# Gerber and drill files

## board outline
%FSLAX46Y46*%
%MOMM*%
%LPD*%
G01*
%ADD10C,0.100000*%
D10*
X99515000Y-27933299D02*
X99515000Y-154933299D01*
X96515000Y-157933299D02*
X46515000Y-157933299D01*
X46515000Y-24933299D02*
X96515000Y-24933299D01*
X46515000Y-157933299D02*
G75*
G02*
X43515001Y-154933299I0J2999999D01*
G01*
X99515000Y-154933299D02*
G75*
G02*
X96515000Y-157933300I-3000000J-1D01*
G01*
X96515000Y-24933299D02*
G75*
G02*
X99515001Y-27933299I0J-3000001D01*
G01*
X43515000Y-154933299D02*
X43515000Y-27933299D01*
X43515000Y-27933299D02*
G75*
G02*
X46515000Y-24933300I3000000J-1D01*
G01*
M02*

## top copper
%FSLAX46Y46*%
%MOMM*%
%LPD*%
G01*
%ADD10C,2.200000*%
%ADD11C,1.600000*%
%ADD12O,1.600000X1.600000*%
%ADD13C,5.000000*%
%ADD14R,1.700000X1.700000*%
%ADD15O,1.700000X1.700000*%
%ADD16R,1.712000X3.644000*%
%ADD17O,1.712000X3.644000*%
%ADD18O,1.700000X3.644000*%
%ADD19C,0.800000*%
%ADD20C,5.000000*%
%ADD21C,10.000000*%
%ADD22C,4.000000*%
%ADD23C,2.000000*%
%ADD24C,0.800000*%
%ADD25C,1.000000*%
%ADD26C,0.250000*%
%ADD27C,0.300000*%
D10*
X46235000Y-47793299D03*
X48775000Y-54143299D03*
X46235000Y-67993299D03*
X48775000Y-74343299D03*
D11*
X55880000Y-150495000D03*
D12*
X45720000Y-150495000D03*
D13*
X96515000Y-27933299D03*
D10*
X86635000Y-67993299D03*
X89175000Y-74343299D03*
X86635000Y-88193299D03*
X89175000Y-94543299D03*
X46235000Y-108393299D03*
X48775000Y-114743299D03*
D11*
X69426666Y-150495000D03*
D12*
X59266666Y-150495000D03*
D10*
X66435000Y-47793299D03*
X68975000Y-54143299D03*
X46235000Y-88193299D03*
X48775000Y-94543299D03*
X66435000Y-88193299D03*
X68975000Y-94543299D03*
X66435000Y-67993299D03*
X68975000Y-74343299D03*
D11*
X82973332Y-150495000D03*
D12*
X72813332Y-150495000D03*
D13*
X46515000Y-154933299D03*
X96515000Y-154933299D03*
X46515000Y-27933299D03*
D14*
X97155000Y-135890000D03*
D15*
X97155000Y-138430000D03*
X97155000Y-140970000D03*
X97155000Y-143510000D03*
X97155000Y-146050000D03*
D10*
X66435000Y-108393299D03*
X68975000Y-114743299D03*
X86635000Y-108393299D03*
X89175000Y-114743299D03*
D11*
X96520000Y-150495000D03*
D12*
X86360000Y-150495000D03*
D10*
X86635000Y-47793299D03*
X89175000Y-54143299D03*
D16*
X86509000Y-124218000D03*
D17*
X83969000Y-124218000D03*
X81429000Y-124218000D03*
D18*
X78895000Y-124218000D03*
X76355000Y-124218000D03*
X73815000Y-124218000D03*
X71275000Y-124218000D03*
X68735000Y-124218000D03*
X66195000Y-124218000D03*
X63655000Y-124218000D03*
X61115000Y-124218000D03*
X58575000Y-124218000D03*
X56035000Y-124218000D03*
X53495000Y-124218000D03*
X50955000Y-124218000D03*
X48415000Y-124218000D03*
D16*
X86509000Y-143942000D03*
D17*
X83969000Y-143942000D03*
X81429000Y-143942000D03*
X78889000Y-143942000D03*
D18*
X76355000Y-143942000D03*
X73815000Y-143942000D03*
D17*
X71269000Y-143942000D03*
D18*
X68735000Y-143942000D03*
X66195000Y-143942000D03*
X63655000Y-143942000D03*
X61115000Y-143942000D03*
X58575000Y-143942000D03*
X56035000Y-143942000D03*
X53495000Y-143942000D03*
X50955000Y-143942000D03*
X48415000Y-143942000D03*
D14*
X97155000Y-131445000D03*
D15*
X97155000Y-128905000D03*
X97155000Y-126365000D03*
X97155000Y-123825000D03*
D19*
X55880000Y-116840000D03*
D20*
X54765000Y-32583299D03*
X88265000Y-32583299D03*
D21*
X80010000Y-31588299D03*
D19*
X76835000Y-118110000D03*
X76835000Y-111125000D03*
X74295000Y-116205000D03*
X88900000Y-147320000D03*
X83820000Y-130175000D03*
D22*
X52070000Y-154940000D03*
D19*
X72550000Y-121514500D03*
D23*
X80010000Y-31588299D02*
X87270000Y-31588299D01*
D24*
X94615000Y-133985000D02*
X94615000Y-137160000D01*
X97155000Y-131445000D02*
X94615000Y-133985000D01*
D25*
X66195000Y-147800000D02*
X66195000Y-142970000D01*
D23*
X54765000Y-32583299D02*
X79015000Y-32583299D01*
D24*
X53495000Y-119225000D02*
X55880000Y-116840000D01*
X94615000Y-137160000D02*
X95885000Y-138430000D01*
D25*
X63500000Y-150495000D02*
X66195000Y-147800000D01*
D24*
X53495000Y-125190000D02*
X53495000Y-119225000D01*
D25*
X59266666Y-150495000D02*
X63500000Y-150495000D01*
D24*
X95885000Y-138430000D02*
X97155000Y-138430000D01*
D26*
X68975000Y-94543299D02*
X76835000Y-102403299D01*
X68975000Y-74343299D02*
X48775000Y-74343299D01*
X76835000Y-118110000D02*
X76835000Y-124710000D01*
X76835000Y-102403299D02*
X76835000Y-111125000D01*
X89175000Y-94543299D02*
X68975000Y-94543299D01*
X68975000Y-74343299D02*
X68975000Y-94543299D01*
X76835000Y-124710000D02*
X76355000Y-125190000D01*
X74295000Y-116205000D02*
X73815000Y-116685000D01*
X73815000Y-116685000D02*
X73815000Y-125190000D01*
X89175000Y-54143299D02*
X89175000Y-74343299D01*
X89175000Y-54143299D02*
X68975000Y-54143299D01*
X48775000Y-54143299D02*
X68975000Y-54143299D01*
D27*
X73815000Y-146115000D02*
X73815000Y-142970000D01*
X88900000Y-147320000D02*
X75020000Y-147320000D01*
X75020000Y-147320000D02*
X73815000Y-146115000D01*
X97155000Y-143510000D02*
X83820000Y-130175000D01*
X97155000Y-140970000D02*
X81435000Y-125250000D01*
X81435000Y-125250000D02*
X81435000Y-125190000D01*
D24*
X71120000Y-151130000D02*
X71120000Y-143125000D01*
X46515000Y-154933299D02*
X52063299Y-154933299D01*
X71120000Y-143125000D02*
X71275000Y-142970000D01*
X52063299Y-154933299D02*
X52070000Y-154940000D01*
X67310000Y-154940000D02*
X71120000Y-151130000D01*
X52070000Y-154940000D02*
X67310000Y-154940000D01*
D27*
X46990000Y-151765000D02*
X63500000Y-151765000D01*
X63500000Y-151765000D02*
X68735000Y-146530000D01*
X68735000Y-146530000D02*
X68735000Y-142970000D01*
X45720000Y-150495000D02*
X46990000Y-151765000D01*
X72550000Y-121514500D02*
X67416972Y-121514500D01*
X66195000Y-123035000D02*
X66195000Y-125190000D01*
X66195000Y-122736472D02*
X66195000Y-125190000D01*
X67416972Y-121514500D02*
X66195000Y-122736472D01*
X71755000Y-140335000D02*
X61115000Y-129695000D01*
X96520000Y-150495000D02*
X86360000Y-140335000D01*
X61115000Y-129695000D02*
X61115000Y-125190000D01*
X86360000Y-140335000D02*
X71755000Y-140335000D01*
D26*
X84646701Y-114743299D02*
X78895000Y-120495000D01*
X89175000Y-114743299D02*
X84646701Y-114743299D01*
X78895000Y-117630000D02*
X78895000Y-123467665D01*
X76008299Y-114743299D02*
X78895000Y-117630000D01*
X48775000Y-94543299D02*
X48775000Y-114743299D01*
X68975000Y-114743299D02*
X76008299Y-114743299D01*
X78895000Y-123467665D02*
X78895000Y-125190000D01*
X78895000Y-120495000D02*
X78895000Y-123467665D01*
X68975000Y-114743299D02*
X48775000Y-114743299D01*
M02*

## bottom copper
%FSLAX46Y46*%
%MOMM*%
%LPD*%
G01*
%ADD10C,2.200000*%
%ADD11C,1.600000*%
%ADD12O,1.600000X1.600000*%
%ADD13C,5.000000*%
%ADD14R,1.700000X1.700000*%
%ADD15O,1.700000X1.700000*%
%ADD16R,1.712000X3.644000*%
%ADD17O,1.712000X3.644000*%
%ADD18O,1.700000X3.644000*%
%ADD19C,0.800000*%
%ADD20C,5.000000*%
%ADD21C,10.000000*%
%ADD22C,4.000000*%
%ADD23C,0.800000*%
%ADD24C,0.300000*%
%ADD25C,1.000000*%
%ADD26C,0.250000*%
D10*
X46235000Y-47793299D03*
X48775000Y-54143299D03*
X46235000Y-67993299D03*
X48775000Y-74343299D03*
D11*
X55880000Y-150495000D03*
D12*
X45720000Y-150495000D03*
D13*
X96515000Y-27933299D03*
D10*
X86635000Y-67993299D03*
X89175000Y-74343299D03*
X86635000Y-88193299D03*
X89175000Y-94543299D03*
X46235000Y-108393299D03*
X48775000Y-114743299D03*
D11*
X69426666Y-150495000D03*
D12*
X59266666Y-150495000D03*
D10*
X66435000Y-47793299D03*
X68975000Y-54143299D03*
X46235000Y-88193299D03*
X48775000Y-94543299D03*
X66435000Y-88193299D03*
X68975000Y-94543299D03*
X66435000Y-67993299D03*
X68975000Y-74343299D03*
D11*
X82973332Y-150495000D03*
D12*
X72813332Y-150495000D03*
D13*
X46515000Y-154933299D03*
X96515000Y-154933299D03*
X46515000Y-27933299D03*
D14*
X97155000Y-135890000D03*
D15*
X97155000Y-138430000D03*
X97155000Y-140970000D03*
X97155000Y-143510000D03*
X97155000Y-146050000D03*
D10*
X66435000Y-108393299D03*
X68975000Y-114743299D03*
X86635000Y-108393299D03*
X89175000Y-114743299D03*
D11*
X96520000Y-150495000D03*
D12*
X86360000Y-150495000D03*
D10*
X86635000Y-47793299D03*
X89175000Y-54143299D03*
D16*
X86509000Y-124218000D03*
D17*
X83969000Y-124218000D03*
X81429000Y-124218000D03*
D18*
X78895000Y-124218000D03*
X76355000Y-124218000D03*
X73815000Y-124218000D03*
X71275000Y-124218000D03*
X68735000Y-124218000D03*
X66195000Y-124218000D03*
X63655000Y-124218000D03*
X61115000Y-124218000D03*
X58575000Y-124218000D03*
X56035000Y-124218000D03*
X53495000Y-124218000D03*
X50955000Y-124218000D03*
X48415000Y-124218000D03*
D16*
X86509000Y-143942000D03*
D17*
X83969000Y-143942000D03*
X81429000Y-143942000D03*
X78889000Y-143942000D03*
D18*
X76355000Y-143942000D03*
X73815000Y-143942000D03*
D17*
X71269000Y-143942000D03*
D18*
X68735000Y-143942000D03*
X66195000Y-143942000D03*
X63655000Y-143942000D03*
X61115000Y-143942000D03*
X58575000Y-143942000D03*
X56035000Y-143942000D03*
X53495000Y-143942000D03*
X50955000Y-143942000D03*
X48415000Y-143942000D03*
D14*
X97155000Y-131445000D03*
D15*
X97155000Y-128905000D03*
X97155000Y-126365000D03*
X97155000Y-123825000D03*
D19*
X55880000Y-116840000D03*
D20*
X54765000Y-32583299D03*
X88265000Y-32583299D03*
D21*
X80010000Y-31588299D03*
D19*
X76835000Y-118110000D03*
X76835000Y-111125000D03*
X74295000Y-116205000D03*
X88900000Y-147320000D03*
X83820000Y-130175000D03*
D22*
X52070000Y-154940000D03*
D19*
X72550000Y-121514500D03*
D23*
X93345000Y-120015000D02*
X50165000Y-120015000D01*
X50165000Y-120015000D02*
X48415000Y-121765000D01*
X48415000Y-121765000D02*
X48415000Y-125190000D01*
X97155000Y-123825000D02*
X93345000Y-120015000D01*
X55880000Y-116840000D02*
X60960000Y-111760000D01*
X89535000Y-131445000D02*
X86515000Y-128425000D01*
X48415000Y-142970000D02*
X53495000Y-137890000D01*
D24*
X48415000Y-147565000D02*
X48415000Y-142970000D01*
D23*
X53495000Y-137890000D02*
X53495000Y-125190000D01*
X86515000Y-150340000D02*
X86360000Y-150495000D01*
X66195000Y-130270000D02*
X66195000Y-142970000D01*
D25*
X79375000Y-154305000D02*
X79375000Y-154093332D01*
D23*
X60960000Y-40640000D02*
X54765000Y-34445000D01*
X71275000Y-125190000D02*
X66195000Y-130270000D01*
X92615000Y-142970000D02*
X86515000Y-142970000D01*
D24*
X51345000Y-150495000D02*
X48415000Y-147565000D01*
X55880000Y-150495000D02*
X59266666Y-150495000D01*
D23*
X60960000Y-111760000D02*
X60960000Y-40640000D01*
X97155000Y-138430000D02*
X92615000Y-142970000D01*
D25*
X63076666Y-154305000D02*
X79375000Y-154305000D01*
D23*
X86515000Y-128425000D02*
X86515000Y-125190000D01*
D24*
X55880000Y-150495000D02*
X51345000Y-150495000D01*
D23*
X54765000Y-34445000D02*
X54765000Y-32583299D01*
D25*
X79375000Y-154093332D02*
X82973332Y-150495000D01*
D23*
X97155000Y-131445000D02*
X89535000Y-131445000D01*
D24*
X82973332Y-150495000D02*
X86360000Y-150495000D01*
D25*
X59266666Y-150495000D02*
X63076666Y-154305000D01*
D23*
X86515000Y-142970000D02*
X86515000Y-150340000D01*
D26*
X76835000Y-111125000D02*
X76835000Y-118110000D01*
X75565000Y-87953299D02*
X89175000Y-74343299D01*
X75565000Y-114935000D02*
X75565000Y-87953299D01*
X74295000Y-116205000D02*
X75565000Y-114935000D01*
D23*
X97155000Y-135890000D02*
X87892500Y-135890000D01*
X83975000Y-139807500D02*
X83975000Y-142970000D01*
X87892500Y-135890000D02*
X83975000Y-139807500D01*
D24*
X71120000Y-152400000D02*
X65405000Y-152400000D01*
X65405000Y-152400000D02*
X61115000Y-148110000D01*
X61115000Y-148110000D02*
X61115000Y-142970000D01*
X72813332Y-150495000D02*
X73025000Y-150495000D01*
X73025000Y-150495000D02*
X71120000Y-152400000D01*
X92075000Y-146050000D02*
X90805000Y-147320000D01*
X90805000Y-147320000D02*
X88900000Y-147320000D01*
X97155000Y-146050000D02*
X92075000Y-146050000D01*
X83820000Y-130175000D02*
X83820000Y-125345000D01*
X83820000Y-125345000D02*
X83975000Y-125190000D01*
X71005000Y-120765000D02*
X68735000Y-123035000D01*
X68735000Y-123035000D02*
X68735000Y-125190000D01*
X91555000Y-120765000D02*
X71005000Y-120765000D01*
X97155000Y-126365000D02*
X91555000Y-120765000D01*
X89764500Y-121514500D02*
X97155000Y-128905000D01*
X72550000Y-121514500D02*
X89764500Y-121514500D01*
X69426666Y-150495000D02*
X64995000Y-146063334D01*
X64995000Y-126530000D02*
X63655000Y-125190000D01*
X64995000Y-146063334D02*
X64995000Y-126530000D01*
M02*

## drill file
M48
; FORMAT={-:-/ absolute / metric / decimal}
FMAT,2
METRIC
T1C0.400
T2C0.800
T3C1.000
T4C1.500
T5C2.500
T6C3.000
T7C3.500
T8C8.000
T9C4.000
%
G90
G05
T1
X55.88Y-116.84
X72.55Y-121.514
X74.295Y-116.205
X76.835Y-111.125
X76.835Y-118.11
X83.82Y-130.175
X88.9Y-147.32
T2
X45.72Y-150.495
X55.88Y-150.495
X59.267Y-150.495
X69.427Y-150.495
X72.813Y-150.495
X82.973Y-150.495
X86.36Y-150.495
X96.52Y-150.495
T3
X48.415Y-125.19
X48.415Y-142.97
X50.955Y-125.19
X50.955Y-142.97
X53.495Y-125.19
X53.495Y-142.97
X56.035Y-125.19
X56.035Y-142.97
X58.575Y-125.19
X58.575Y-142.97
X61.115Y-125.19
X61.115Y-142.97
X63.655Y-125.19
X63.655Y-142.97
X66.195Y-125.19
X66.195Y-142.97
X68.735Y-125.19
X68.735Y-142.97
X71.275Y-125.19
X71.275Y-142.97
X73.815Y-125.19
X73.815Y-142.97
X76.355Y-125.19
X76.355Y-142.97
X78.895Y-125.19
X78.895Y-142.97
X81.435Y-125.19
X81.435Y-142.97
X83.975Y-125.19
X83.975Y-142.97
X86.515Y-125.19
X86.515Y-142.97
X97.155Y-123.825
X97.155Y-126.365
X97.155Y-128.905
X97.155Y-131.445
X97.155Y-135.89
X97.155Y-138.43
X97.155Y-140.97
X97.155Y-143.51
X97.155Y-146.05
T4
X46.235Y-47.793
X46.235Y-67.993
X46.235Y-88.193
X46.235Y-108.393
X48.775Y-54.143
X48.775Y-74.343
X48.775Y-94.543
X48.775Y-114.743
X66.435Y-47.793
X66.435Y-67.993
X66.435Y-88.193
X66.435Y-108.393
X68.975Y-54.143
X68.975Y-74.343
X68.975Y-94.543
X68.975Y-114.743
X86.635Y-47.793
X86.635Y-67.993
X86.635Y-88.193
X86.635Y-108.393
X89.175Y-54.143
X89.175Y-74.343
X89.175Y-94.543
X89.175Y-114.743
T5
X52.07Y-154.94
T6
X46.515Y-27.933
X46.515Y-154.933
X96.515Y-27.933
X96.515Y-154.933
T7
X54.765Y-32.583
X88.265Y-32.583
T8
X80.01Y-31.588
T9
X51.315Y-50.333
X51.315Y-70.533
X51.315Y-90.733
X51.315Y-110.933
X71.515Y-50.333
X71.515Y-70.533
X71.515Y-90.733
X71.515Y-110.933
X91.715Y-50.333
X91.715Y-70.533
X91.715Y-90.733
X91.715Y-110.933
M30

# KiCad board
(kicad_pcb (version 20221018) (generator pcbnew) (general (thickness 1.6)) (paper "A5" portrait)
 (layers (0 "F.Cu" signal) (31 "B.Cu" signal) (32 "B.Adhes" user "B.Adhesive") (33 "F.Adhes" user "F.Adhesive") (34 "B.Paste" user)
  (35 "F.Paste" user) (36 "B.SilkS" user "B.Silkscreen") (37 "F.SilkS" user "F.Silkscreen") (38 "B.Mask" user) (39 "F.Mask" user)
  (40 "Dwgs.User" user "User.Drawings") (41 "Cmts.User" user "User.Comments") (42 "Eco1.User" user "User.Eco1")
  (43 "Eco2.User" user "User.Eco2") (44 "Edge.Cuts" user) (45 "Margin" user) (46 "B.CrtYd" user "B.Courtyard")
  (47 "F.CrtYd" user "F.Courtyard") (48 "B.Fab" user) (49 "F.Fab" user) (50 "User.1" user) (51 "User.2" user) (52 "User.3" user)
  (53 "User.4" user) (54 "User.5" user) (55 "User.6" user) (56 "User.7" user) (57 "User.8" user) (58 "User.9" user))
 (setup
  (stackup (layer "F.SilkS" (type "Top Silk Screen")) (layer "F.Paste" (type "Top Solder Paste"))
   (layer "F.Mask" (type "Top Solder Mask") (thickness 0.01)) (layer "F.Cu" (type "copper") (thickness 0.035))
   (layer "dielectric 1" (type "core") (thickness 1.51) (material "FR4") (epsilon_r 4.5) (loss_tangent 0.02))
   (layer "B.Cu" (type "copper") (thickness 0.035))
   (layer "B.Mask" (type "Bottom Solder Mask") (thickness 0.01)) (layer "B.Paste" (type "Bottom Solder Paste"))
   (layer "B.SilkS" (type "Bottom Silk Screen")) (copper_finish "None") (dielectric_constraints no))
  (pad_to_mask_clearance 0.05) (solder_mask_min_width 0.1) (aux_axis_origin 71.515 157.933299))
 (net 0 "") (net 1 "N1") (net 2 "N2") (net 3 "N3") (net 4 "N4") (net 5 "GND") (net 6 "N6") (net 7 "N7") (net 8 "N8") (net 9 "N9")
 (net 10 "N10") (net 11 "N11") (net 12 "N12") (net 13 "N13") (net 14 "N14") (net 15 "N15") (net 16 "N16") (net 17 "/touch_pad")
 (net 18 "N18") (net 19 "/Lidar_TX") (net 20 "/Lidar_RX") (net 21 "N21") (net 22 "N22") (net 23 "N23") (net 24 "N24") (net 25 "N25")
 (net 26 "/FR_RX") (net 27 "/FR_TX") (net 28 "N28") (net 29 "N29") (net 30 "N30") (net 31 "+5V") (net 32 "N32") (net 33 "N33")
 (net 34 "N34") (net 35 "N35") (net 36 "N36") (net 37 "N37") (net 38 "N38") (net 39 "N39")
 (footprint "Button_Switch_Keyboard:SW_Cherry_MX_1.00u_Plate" (layer "F.Cu") (at 46.235 47.793299 90)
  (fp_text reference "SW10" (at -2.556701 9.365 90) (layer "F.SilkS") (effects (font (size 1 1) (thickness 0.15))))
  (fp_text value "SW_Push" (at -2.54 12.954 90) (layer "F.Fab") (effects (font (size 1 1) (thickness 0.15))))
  (pad "" np_thru_hole circle (at -2.54 5.08 90) (size 4 4) (drill 4) (layers "*.Cu" "*.Mask"))
  (pad "1" thru_hole circle (at 0 0 90) (size 2.2 2.2) (drill 1.5) (layers "*.Cu" "*.Mask") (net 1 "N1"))
  (pad "2" thru_hole circle (at -6.35 2.54 90) (size 2.2 2.2) (drill 1.5) (layers "*.Cu" "*.Mask") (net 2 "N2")))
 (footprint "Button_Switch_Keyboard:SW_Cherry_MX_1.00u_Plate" (layer "F.Cu") (at 46.235 67.993299 90)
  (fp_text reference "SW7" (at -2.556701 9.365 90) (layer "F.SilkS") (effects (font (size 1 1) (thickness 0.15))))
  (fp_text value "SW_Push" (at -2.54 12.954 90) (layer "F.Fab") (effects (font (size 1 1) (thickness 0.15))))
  (pad "" np_thru_hole circle (at -2.54 5.08 90) (size 4 4) (drill 4) (layers "*.Cu" "*.Mask"))
  (pad "1" thru_hole circle (at 0 0 90) (size 2.2 2.2) (drill 1.5) (layers "*.Cu" "*.Mask") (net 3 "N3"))
  (pad "2" thru_hole circle (at -6.35 2.54 90) (size 2.2 2.2) (drill 1.5) (layers "*.Cu" "*.Mask") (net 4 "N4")))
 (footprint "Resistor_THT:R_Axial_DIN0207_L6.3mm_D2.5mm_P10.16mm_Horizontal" (layer "F.Cu") (at 55.88 150.495 180)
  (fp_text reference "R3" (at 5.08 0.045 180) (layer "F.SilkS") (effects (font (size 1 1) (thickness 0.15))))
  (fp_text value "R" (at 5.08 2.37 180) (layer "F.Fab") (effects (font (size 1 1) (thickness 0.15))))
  (pad "1" thru_hole circle (at 0 0 180) (size 1.6 1.6) (drill 0.8) (layers "*.Cu" "*.Mask") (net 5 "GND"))
  (pad "2" thru_hole oval (at 10.16 0 180) (size 1.6 1.6) (drill 0.8) (layers "*.Cu" "*.Mask") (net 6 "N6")))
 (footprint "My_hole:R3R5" (layer "F.Cu") (at 96.52 27.763299)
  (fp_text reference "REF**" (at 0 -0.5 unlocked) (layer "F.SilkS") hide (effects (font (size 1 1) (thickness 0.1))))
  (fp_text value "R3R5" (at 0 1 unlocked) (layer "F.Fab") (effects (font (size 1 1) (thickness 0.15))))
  (pad "1" thru_hole circle (at -0.005 0.17 180) (size 5 5) (drill 3) (layers "*.Cu" "*.Mask") (remove_unused_layers) (keep_end_layers)
   (zone_layer_connections)))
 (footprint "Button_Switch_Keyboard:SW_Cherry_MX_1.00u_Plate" (layer "F.Cu") (at 86.635 67.993299 90)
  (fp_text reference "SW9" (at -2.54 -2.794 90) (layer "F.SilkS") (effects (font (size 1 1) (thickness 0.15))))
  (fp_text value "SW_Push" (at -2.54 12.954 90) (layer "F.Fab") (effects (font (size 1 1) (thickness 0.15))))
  (pad "" np_thru_hole circle (at -2.54 5.08 90) (size 4 4) (drill 4) (layers "*.Cu" "*.Mask"))
  (pad "1" thru_hole circle (at 0 0 90) (size 2.2 2.2) (drill 1.5) (layers "*.Cu" "*.Mask") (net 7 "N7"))
  (pad "2" thru_hole circle (at -6.35 2.54 90) (size 2.2 2.2) (drill 1.5) (layers "*.Cu" "*.Mask") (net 2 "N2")))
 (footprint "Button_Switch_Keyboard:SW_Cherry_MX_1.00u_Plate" (layer "F.Cu") (at 86.635 88.193299 90)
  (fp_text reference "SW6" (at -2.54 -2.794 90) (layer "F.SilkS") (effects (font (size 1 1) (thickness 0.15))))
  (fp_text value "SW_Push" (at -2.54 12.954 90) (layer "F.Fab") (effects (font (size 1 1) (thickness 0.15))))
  (pad "" np_thru_hole circle (at -2.54 5.08 90) (size 4 4) (drill 4) (layers "*.Cu" "*.Mask"))
  (pad "1" thru_hole circle (at 0 0 90) (size 2.2 2.2) (drill 1.5) (layers "*.Cu" "*.Mask") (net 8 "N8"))
  (pad "2" thru_hole circle (at -6.35 2.54 90) (size 2.2 2.2) (drill 1.5) (layers "*.Cu" "*.Mask") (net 4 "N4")))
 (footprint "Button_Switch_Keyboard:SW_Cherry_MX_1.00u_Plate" (layer "F.Cu") (at 46.235 108.393299 90)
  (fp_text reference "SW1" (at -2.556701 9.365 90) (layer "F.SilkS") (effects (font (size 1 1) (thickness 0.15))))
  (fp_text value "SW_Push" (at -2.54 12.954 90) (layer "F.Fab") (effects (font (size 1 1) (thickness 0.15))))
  (pad "" np_thru_hole circle (at -2.54 5.08 90) (size 4 4) (drill 4) (layers "*.Cu" "*.Mask"))
  (pad "1" thru_hole circle (at 0 0 90) (size 2.2 2.2) (drill 1.5) (layers "*.Cu" "*.Mask") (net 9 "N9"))
  (pad "2" thru_hole circle (at -6.35 2.54 90) (size 2.2 2.2) (drill 1.5) (layers "*.Cu" "*.Mask") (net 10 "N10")))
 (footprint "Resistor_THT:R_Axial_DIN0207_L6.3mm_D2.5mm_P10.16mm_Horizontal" (layer "F.Cu") (at 69.426666 150.495 180)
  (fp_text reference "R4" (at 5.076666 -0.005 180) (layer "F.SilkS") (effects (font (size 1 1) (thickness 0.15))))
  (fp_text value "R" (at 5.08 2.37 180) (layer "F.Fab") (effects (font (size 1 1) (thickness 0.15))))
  (pad "1" thru_hole circle (at 0 0 180) (size 1.6 1.6) (drill 0.8) (layers "*.Cu" "*.Mask") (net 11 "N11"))
  (pad "2" thru_hole oval (at 10.16 0 180) (size 1.6 1.6) (drill 0.8) (layers "*.Cu" "*.Mask") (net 5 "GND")))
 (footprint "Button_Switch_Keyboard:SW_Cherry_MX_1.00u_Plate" (layer "F.Cu") (at 66.435 47.793299 90)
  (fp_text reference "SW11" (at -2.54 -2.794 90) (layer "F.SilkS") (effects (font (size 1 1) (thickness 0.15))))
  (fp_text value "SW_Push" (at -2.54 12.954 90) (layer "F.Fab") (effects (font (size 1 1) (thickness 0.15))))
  (pad "" np_thru_hole circle (at -2.54 5.08 90) (size 4 4) (drill 4) (layers "*.Cu" "*.Mask"))
  (pad "1" thru_hole circle (at 0 0 90) (size 2.2 2.2) (drill 1.5) (layers "*.Cu" "*.Mask") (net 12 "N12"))
  (pad "2" thru_hole circle (at -6.35 2.54 90) (size 2.2 2.2) (drill 1.5) (layers "*.Cu" "*.Mask") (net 2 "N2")))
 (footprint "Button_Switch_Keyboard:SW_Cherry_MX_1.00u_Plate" (layer "F.Cu") (at 46.235 88.193299 90)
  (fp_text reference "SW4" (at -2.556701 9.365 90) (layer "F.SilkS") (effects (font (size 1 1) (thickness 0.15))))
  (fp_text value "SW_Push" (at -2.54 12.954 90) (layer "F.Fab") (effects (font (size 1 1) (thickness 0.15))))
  (pad "" np_thru_hole circle (at -2.54 5.08 90) (size 4 4) (drill 4) (layers "*.Cu" "*.Mask"))
  (pad "1" thru_hole circle (at 0 0 90) (size 2.2 2.2) (drill 1.5) (layers "*.Cu" "*.Mask") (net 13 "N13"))
  (pad "2" thru_hole circle (at -6.35 2.54 90) (size 2.2 2.2) (drill 1.5) (layers "*.Cu" "*.Mask") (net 10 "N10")))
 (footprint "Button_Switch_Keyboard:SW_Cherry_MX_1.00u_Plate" (layer "F.Cu") (at 66.435 88.193299 90)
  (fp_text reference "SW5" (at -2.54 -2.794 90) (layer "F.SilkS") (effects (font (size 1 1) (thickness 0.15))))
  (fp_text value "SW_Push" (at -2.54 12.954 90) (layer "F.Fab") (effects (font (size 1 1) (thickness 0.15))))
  (pad "" np_thru_hole circle (at -2.54 5.08 90) (size 4 4) (drill 4) (layers "*.Cu" "*.Mask"))
  (pad "1" thru_hole circle (at 0 0 90) (size 2.2 2.2) (drill 1.5) (layers "*.Cu" "*.Mask") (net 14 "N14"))
  (pad "2" thru_hole circle (at -6.35 2.54 90) (size 2.2 2.2) (drill 1.5) (layers "*.Cu" "*.Mask") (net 4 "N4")))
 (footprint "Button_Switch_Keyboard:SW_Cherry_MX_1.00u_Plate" (layer "F.Cu") (at 66.435 67.993299 90)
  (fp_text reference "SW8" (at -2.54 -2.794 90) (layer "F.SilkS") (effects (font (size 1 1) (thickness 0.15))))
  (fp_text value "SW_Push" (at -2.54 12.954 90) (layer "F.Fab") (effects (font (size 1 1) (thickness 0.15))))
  (pad "" np_thru_hole circle (at -2.54 5.08 90) (size 4 4) (drill 4) (layers "*.Cu" "*.Mask"))
  (pad "1" thru_hole circle (at 0 0 90) (size 2.2 2.2) (drill 1.5) (layers "*.Cu" "*.Mask") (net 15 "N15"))
  (pad "2" thru_hole circle (at -6.35 2.54 90) (size 2.2 2.2) (drill 1.5) (layers "*.Cu" "*.Mask") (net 4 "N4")))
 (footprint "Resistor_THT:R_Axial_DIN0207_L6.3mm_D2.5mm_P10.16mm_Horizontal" (layer "F.Cu") (at 82.973332 150.495 180)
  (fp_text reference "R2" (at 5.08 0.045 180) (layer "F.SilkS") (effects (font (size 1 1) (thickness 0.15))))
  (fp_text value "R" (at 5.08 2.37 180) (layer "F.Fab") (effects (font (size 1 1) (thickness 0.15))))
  (pad "1" thru_hole circle (at 0 0 180) (size 1.6 1.6) (drill 0.8) (layers "*.Cu" "*.Mask") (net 5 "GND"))
  (pad "2" thru_hole oval (at 10.16 0 180) (size 1.6 1.6) (drill 0.8) (layers "*.Cu" "*.Mask") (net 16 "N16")))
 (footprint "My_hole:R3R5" (layer "F.Cu") (at 46.99 154.763299)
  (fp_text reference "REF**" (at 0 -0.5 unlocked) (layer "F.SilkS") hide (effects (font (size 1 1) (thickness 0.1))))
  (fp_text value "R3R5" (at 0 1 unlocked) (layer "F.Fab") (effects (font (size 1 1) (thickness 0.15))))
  (pad "1" thru_hole circle (at -0.475 0.17 180) (size 5 5) (drill 3) (layers "*.Cu" "*.Mask") (remove_unused_layers) (keep_end_layers)
   (zone_layer_connections) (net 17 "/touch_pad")))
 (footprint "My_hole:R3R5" (layer "F.Cu") (at 96.52 155.398299)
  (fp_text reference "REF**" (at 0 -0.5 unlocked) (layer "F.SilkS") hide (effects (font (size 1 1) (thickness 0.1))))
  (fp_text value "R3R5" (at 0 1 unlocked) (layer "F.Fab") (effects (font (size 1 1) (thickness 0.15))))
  (pad "1" thru_hole circle (at -0.005 -0.465 180) (size 5 5) (drill 3) (layers "*.Cu" "*.Mask") (remove_unused_layers) (keep_end_layers)
   (zone_layer_connections)))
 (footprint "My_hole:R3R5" (layer "F.Cu") (at 46.355 27.763299)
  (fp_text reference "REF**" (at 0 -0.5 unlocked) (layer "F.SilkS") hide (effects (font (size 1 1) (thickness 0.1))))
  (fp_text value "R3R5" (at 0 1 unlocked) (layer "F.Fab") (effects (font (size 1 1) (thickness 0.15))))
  (pad "1" thru_hole circle (at 0.16 0.17 180) (size 5 5) (drill 3) (layers "*.Cu" "*.Mask") (remove_unused_layers) (keep_end_layers)
   (zone_layer_connections)))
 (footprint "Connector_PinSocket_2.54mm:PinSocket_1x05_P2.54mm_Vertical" (layer "F.Cu") (at 97.155 135.89)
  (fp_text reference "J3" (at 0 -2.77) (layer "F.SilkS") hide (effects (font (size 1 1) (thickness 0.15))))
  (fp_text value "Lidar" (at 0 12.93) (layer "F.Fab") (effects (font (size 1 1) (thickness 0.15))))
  (pad "1" thru_hole rect (at 0 0) (size 1.7 1.7) (drill 1) (layers "*.Cu" "*.Mask") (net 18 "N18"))
  (pad "2" thru_hole oval (at 0 2.54) (size 1.7 1.7) (drill 1) (layers "*.Cu" "*.Mask") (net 5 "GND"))
  (pad "3" thru_hole oval (at 0 5.08) (size 1.7 1.7) (drill 1) (layers "*.Cu" "*.Mask") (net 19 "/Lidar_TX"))
  (pad "4" thru_hole oval (at 0 7.62) (size 1.7 1.7) (drill 1) (layers "*.Cu" "*.Mask") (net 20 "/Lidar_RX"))
  (pad "5" thru_hole oval (at 0 10.16) (size 1.7 1.7) (drill 1) (layers "*.Cu" "*.Mask") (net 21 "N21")))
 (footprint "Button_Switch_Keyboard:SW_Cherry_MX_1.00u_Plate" (layer "F.Cu") (at 66.435 108.393299 90)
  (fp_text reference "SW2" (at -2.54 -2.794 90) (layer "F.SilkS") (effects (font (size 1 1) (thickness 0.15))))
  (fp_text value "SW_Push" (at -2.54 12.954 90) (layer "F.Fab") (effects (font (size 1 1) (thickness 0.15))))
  (pad "" np_thru_hole circle (at -2.54 5.08 90) (size 4 4) (drill 4) (layers "*.Cu" "*.Mask"))
  (pad "1" thru_hole circle (at 0 0 90) (size 2.2 2.2) (drill 1.5) (layers "*.Cu" "*.Mask") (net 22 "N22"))
  (pad "2" thru_hole circle (at -6.35 2.54 90) (size 2.2 2.2) (drill 1.5) (layers "*.Cu" "*.Mask") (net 10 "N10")))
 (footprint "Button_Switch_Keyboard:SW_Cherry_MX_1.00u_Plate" (layer "F.Cu") (at 86.635 108.393299 90)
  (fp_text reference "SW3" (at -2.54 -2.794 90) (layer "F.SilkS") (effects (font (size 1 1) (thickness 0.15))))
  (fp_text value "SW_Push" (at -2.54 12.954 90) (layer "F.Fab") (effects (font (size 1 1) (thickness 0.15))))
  (pad "" np_thru_hole circle (at -2.54 5.08 90) (size 4 4) (drill 4) (layers "*.Cu" "*.Mask"))
  (pad "1" thru_hole circle (at 0 0 90) (size 2.2 2.2) (drill 1.5) (layers "*.Cu" "*.Mask") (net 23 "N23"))
  (pad "2" thru_hole circle (at -6.35 2.54 90) (size 2.2 2.2) (drill 1.5) (layers "*.Cu" "*.Mask") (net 10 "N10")))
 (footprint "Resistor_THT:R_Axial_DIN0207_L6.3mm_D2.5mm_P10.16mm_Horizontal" (layer "F.Cu") (at 96.52 150.495 180)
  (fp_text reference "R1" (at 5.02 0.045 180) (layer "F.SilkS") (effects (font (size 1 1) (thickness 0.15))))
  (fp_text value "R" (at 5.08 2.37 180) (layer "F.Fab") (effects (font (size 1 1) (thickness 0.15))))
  (pad "1" thru_hole circle (at 0 0 180) (size 1.6 1.6) (drill 0.8) (layers "*.Cu" "*.Mask") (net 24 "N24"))
  (pad "2" thru_hole oval (at 10.16 0 180) (size 1.6 1.6) (drill 0.8) (layers "*.Cu" "*.Mask") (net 5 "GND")))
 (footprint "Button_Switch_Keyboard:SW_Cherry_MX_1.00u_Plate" (layer "F.Cu") (at 86.635 47.793299 90)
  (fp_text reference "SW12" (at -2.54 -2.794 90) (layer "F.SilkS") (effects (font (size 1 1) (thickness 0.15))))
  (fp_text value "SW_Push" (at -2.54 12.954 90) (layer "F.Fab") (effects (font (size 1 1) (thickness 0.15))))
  (pad "" np_thru_hole circle (at -2.54 5.08 90) (size 4 4) (drill 4) (layers "*.Cu" "*.Mask"))
  (pad "1" thru_hole circle (at 0 0 90) (size 2.2 2.2) (drill 1.5) (layers "*.Cu" "*.Mask") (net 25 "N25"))
  (pad "2" thru_hole circle (at -6.35 2.54 90) (size 2.2 2.2) (drill 1.5) (layers "*.Cu" "*.Mask") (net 2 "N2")))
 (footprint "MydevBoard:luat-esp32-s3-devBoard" (layer "F.Cu") (at 41.965 134.08 -90)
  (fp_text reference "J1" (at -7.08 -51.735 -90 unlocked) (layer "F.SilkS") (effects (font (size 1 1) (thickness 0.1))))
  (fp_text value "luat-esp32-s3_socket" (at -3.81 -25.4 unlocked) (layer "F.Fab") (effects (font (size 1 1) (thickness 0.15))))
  (pad "1" thru_hole rect (at -8.89 -44.55 270) (size 3.644 1.712) (drill 1 (offset -0.972 0.006)) (layers "*.Cu" "*.Mask") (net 5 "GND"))
  (pad "2" thru_hole oval (at -8.89 -42.01 270) (size 3.644 1.712) (drill 1 (offset -0.972 0.006)) (layers "*.Cu" "*.Mask")
   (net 20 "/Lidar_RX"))
  (pad "3" thru_hole oval (at -8.89 -39.47 270) (size 3.644 1.712) (drill 1 (offset -0.972 0.006)) (layers "*.Cu" "*.Mask")
   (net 19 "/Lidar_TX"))
  (pad "4" thru_hole oval (at -8.89 -36.93 270) (size 3.644 1.7) (drill 1 (offset -0.972 0)) (layers "*.Cu" "*.Mask") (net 10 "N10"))
  (pad "5" thru_hole oval (at -8.89 -34.39 270) (size 3.644 1.7) (drill 1 (offset -0.972 0)) (layers "*.Cu" "*.Mask") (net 4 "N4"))
  (pad "6" thru_hole oval (at -8.89 -31.85 270) (size 3.644 1.7) (drill 1 (offset -0.972 0)) (layers "*.Cu" "*.Mask") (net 2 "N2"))
  (pad "7" thru_hole oval (at -8.89 -29.31 270) (size 3.644 1.7) (drill 1 (offset -0.972 0)) (layers "*.Cu" "*.Mask") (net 5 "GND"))
  (pad "8" thru_hole oval (at -8.89 -26.77 270) (size 3.644 1.7) (drill 1 (offset -0.972 0)) (layers "*.Cu" "*.Mask") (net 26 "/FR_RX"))
  (pad "9" thru_hole oval (at -8.89 -24.23 270) (size 3.644 1.7) (drill 1 (offset -0.972 0)) (layers "*.Cu" "*.Mask") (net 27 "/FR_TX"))
  (pad "10" thru_hole oval (at -8.89 -21.69 270) (size 3.644 1.7) (drill 1 (offset -0.972 0)) (layers "*.Cu" "*.Mask") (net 11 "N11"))
  (pad "11" thru_hole oval (at -8.89 -19.15 270) (size 3.644 1.7) (drill 1 (offset -0.972 0)) (layers "*.Cu" "*.Mask") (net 24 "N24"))
  (pad "12" thru_hole oval (at -8.89 -16.61 270) (size 3.644 1.7) (drill 1 (offset -0.972 0)) (layers "*.Cu" "*.Mask") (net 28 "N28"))
  (pad "13" thru_hole oval (at -8.89 -14.07 270) (size 3.644 1.7) (drill 1 (offset -0.972 0)) (layers "*.Cu" "*.Mask") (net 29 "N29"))
  (pad "14" thru_hole oval (at -8.89 -11.53 270) (size 3.644 1.7) (drill 1 (offset -0.972 0)) (layers "*.Cu" "*.Mask") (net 5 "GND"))
  (pad "15" thru_hole oval (at -8.89 -8.99 270) (size 3.644 1.7) (drill 1 (offset -0.972 0)) (layers "*.Cu" "*.Mask") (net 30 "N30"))
  (pad "16" thru_hole oval (at -8.89 -6.45 270) (size 3.644 1.7) (drill 1 (offset -0.972 0)) (layers "*.Cu" "*.Mask") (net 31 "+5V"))
  (pad "17" thru_hole rect (at 8.89 -44.55 270) (size 3.644 1.712) (drill 1 (offset 0.972 0.006)) (layers "*.Cu" "*.Mask") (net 5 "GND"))
  (pad "18" thru_hole oval (at 8.89 -42.01 270) (size 3.644 1.712) (drill 1 (offset 0.972 0.006)) (layers "*.Cu" "*.Mask") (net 18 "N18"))
  (pad "19" thru_hole oval (at 8.89 -39.47 270) (size 3.644 1.712) (drill 1 (offset 0.972 0.006)) (layers "*.Cu" "*.Mask") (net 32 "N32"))
  (pad "20" thru_hole oval (at 8.89 -36.93 270) (size 3.644 1.712) (drill 1 (offset 0.972 0.006)) (layers "*.Cu" "*.Mask") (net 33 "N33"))
  (pad "21" thru_hole oval (at 8.89 -34.39 270) (size 3.644 1.7) (drill 1 (offset 0.972 0)) (layers "*.Cu" "*.Mask") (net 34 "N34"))
  (pad "22" thru_hole oval (at 8.89 -31.85 270) (size 3.644 1.7) (drill 1 (offset 0.972 0)) (layers "*.Cu" "*.Mask") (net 21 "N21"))
  (pad "23" thru_hole oval (at 8.89 -29.31 270) (size 3.644 1.712) (drill 1 (offset 0.972 0.006)) (layers "*.Cu" "*.Mask")
   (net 17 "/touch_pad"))
  (pad "24" thru_hole oval (at 8.89 -26.77 270) (size 3.644 1.7) (drill 1 (offset 0.972 0)) (layers "*.Cu" "*.Mask") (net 6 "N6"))
  (pad "25" thru_hole oval (at 8.89 -24.23 270) (size 3.644 1.7) (drill 1 (offset 0.972 0)) (layers "*.Cu" "*.Mask") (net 5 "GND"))
  (pad "26" thru_hole oval (at 8.89 -21.69 270) (size 3.644 1.7) (drill 1 (offset 0.972 0)) (layers "*.Cu" "*.Mask") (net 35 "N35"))
  (pad "27" thru_hole oval (at 8.89 -19.15 270) (size 3.644 1.7) (drill 1 (offset 0.972 0)) (layers "*.Cu" "*.Mask") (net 16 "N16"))
  (pad "28" thru_hole oval (at 8.89 -16.61 270) (size 3.644 1.7) (drill 1 (offset 0.972 0)) (layers "*.Cu" "*.Mask") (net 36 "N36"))
  (pad "29" thru_hole oval (at 8.89 -14.07 270) (size 3.644 1.7) (drill 1 (offset 0.972 0)) (layers "*.Cu" "*.Mask") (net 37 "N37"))
  (pad "30" thru_hole oval (at 8.89 -11.53 270) (size 3.644 1.7) (drill 1 (offset 0.972 0)) (layers "*.Cu" "*.Mask") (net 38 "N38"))
  (pad "31" thru_hole oval (at 8.89 -8.99 270) (size 3.644 1.7) (drill 1 (offset 0.972 0)) (layers "*.Cu" "*.Mask") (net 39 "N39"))
  (pad "32" thru_hole oval (at 8.89 -6.45 270) (size 3.644 1.7) (drill 1 (offset 0.972 0)) (layers "*.Cu" "*.Mask") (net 5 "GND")))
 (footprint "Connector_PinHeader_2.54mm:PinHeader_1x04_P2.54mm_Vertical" (layer "B.Cu") (at 97.155 131.445)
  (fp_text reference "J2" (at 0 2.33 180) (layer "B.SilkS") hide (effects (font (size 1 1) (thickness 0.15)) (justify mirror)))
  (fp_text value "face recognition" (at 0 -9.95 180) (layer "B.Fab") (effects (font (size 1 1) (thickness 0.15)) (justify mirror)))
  (pad "1" thru_hole rect (at 0 0) (size 1.7 1.7) (drill 1) (layers "*.Cu" "*.Mask") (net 5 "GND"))
  (pad "2" thru_hole oval (at 0 -2.54) (size 1.7 1.7) (drill 1) (layers "*.Cu" "*.Mask") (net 27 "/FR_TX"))
  (pad "3" thru_hole oval (at 0 -5.08) (size 1.7 1.7) (drill 1) (layers "*.Cu" "*.Mask") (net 26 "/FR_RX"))
  (pad "4" thru_hole oval (at 0 -7.62) (size 1.7 1.7) (drill 1) (layers "*.Cu" "*.Mask") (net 31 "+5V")))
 (gr_line (start 99.515 27.933299) (end 99.515 154.933299) (stroke (width 0.1) (type default)) (layer "Edge.Cuts"))
 (gr_line (start 96.515 157.933299) (end 46.515 157.933299) (stroke (width 0.1) (type default)) (layer "Edge.Cuts"))
 (gr_line (start 46.515 24.933299) (end 96.515 24.933299) (stroke (width 0.1) (type default)) (layer "Edge.Cuts"))
 (gr_arc (start 46.515 157.933299) (mid 44.39368 157.054619) (end 43.515 154.933299) (stroke (width 0.1) (type default)) (layer "Edge.Cuts"))
 (gr_arc (start 99.515 154.933299) (mid 98.63632 157.054619) (end 96.515 157.933299) (stroke (width 0.1) (type default)) (layer "Edge.Cuts"))
 (gr_arc (start 96.515 24.933299) (mid 98.63632 25.811979) (end 99.515 27.933299) (stroke (width 0.1) (type default)) (layer "Edge.Cuts"))
 (gr_line (start 43.515 154.933299) (end 43.515 27.933299) (stroke (width 0.1) (type default)) (layer "Edge.Cuts"))
 (gr_arc (start 43.515 27.933299) (mid 44.39368 25.811979) (end 46.515 24.933299) (stroke (width 0.1) (type default)) (layer "Edge.Cuts"))
 (segment (start 93.345 120.015) (end 50.165 120.015) (width 0.8) (layer "B.Cu") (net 31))
 (segment (start 50.165 120.015) (end 48.415 121.765) (width 0.8) (layer "B.Cu") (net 31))
 (segment (start 48.415 121.765) (end 48.415 125.19) (width 0.8) (layer "B.Cu") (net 31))
 (segment (start 97.155 123.825) (end 93.345 120.015) (width 0.8) (layer "B.Cu") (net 31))
 (segment (start 80.01 31.588299) (end 87.27 31.588299) (width 2) (layer "F.Cu") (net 5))
 (segment (start 94.615 133.985) (end 94.615 137.16) (width 0.8) (layer "F.Cu") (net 5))
 (segment (start 97.155 131.445) (end 94.615 133.985) (width 0.8) (layer "F.Cu") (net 5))
 (segment (start 66.195 147.8) (end 66.195 142.97) (width 1) (layer "F.Cu") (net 5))
 (segment (start 54.765 32.583299) (end 79.015 32.583299) (width 2) (layer "F.Cu") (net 5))
 (segment (start 53.495 119.225) (end 55.88 116.84) (width 0.8) (layer "F.Cu") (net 5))
 (segment (start 94.615 137.16) (end 95.885 138.43) (width 0.8) (layer "F.Cu") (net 5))
 (segment (start 63.5 150.495) (end 66.195 147.8) (width 1) (layer "F.Cu") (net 5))
 (segment (start 53.495 125.19) (end 53.495 119.225) (width 0.8) (layer "F.Cu") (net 5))
 (segment (start 59.266666 150.495) (end 63.5 150.495) (width 1) (layer "F.Cu") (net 5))
 (segment (start 95.885 138.43) (end 97.155 138.43) (width 0.8) (layer "F.Cu") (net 5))
 (via (at 55.88 116.84) (size 0.8) (drill 0.4) (layers "F.Cu" "B.Cu") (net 5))
 (via (at 54.765 32.583299) (size 5) (drill 3.5) (layers "F.Cu" "B.Cu") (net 5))
 (via (at 88.265 32.583299) (size 5) (drill 3.5) (layers "F.Cu" "B.Cu") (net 5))
 (via (at 80.01 31.588299) (size 10) (drill 8) (layers "F.Cu" "B.Cu") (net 5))
 (segment (start 55.88 116.84) (end 60.96 111.76) (width 0.8) (layer "B.Cu") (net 5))
 (segment (start 89.535 131.445) (end 86.515 128.425) (width 0.8) (layer "B.Cu") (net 5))
 (segment (start 48.415 142.97) (end 53.495 137.89) (width 0.8) (layer "B.Cu") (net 5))
 (segment (start 48.415 147.565) (end 48.415 142.97) (width 0.3) (layer "B.Cu") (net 5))
 (segment (start 53.495 137.89) (end 53.495 125.19) (width 0.8) (layer "B.Cu") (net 5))
 (segment (start 86.515 150.34) (end 86.36 150.495) (width 0.8) (layer "B.Cu") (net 5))
 (segment (start 66.195 130.27) (end 66.195 142.97) (width 0.8) (layer "B.Cu") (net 5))
 (segment (start 79.375 154.305) (end 79.375 154.093332) (width 1) (layer "B.Cu") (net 5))
 (segment (start 60.96 40.64) (end 54.765 34.445) (width 0.8) (layer "B.Cu") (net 5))
 (segment (start 71.275 125.19) (end 66.195 130.27) (width 0.8) (layer "B.Cu") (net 5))
 (segment (start 92.615 142.97) (end 86.515 142.97) (width 0.8) (layer "B.Cu") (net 5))
 (segment (start 51.345 150.495) (end 48.415 147.565) (width 0.3) (layer "B.Cu") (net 5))
 (segment (start 55.88 150.495) (end 59.266666 150.495) (width 0.3) (layer "B.Cu") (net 5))
 (segment (start 60.96 111.76) (end 60.96 40.64) (width 0.8) (layer "B.Cu") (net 5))
 (segment (start 97.155 138.43) (end 92.615 142.97) (width 0.8) (layer "B.Cu") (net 5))
 (segment (start 63.076666 154.305) (end 79.375 154.305) (width 1) (layer "B.Cu") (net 5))
 (segment (start 86.515 128.425) (end 86.515 125.19) (width 0.8) (layer "B.Cu") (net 5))
 (segment (start 55.88 150.495) (end 51.345 150.495) (width 0.3) (layer "B.Cu") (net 5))
 (segment (start 54.765 34.445) (end 54.765 32.583299) (width 0.8) (layer "B.Cu") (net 5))
 (segment (start 79.375 154.093332) (end 82.973332 150.495) (width 1) (layer "B.Cu") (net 5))
 (segment (start 97.155 131.445) (end 89.535 131.445) (width 0.8) (layer "B.Cu") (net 5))
 (segment (start 82.973332 150.495) (end 86.36 150.495) (width 0.3) (layer "B.Cu") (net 5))
 (segment (start 59.266666 150.495) (end 63.076666 154.305) (width 1) (layer "B.Cu") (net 5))
 (segment (start 86.515 142.97) (end 86.515 150.34) (width 0.8) (layer "B.Cu") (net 5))
 (segment (start 68.975 94.543299) (end 76.835 102.403299) (width 0.25) (layer "F.Cu") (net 4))
 (segment (start 68.975 74.343299) (end 48.775 74.343299) (width 0.25) (layer "F.Cu") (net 4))
 (segment (start 76.835 118.11) (end 76.835 124.71) (width 0.25) (layer "F.Cu") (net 4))
 (segment (start 76.835 102.403299) (end 76.835 111.125) (width 0.25) (layer "F.Cu") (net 4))
 (segment (start 89.175 94.543299) (end 68.975 94.543299) (width 0.25) (layer "F.Cu") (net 4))
 (segment (start 68.975 74.343299) (end 68.975 94.543299) (width 0.25) (layer "F.Cu") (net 4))
 (segment (start 76.835 124.71) (end 76.355 125.19) (width 0.25) (layer "F.Cu") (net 4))
 (via (at 76.835 118.11) (size 0.8) (drill 0.4) (layers "F.Cu" "B.Cu") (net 4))
 (via (at 76.835 111.125) (size 0.8) (drill 0.4) (layers "F.Cu" "B.Cu") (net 4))
 (segment (start 76.835 111.125) (end 76.835 118.11) (width 0.25) (layer "B.Cu") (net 4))
 (segment (start 74.295 116.205) (end 73.815 116.685) (width 0.25) (layer "F.Cu") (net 2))
 (segment (start 73.815 116.685) (end 73.815 125.19) (width 0.25) (layer "F.Cu") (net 2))
 (segment (start 89.175 54.143299) (end 89.175 74.343299) (width 0.25) (layer "F.Cu") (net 2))
 (segment (start 89.175 54.143299) (end 68.975 54.143299) (width 0.25) (layer "F.Cu") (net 2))
 (segment (start 48.775 54.143299) (end 68.975 54.143299) (width 0.25) (layer "F.Cu") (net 2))
 (via (at 74.295 116.205) (size 0.8) (drill 0.4) (layers "F.Cu" "B.Cu") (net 2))
 (segment (start 75.565 87.953299) (end 89.175 74.343299) (width 0.25) (layer "B.Cu") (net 2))
 (segment (start 75.565 114.935) (end 75.565 87.953299) (width 0.25) (layer "B.Cu") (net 2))
 (segment (start 74.295 116.205) (end 75.565 114.935) (width 0.25) (layer "B.Cu") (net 2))
 (segment (start 97.155 135.89) (end 87.8925 135.89) (width 0.8) (layer "B.Cu") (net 18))
 (segment (start 83.975 139.8075) (end 83.975 142.97) (width 0.8) (layer "B.Cu") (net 18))
 (segment (start 87.8925 135.89) (end 83.975 139.8075) (width 0.8) (layer "B.Cu") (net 18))
 (segment (start 71.12 152.4) (end 65.405 152.4) (width 0.3) (layer "B.Cu") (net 16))
 (segment (start 65.405 152.4) (end 61.115 148.11) (width 0.3) (layer "B.Cu") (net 16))
 (segment (start 61.115 148.11) (end 61.115 142.97) (width 0.3) (layer "B.Cu") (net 16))
 (segment (start 72.813332 150.495) (end 73.025 150.495) (width 0.3) (layer "B.Cu") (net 16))
 (segment (start 73.025 150.495) (end 71.12 152.4) (width 0.3) (layer "B.Cu") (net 16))
 (segment (start 73.815 146.115) (end 73.815 142.97) (width 0.3) (layer "F.Cu") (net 21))
 (segment (start 88.9 147.32) (end 75.02 147.32) (width 0.3) (layer "F.Cu") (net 21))
 (segment (start 75.02 147.32) (end 73.815 146.115) (width 0.3) (layer "F.Cu") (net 21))
 (via (at 88.9 147.32) (size 0.8) (drill 0.4) (layers "F.Cu" "B.Cu") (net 21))
 (segment (start 92.075 146.05) (end 90.805 147.32) (width 0.3) (layer "B.Cu") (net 21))
 (segment (start 90.805 147.32) (end 88.9 147.32) (width 0.3) (layer "B.Cu") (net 21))
 (segment (start 97.155 146.05) (end 92.075 146.05) (width 0.3) (layer "B.Cu") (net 21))
 (segment (start 97.155 143.51) (end 83.82 130.175) (width 0.3) (layer "F.Cu") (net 20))
 (via (at 83.82 130.175) (size 0.8) (drill 0.4) (layers "F.Cu" "B.Cu") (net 20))
 (segment (start 83.82 130.175) (end 83.82 125.345) (width 0.3) (layer "B.Cu") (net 20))
 (segment (start 83.82 125.345) (end 83.975 125.19) (width 0.3) (layer "B.Cu") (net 20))
 (segment (start 97.155 140.97) (end 81.435 125.25) (width 0.3) (layer "F.Cu") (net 19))
 (segment (start 81.435 125.25) (end 81.435 125.19) (width 0.3) (layer "F.Cu") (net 19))
 (segment (start 71.12 151.13) (end 71.12 143.125) (width 0.8) (layer "F.Cu") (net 17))
 (segment (start 46.515 154.933299) (end 52.063299 154.933299) (width 0.8) (layer "F.Cu") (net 17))
 (segment (start 71.12 143.125) (end 71.275 142.97) (width 0.8) (layer "F.Cu") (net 17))
 (segment (start 52.063299 154.933299) (end 52.07 154.94) (width 0.8) (layer "F.Cu") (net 17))
 (segment (start 67.31 154.94) (end 71.12 151.13) (width 0.8) (layer "F.Cu") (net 17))
 (segment (start 52.07 154.94) (end 67.31 154.94) (width 0.8) (layer "F.Cu") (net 17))
 (via (at 52.07 154.94) (size 4) (drill 2.5) (layers "F.Cu" "B.Cu") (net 17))
 (segment (start 71.005 120.765) (end 68.735 123.035) (width 0.3) (layer "B.Cu") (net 26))
 (segment (start 68.735 123.035) (end 68.735 125.19) (width 0.3) (layer "B.Cu") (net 26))
 (segment (start 91.555 120.765) (end 71.005 120.765) (width 0.3) (layer "B.Cu") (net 26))
 (segment (start 97.155 126.365) (end 91.555 120.765) (width 0.3) (layer "B.Cu") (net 26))
 (segment (start 46.99 151.765) (end 63.5 151.765) (width 0.3) (layer "F.Cu") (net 6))
 (segment (start 63.5 151.765) (end 68.735 146.53) (width 0.3) (layer "F.Cu") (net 6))
 (segment (start 68.735 146.53) (end 68.735 142.97) (width 0.3) (layer "F.Cu") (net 6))
 (segment (start 45.72 150.495) (end 46.99 151.765) (width 0.3) (layer "F.Cu") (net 6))
 (segment (start 72.55 121.5145) (end 67.416972 121.5145) (width 0.3) (layer "F.Cu") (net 27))
 (segment (start 66.195 123.035) (end 66.195 125.19) (width 0.3) (layer "F.Cu") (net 27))
 (segment (start 66.195 122.736472) (end 66.195 125.19) (width 0.3) (layer "F.Cu") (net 27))
 (segment (start 67.416972 121.5145) (end 66.195 122.736472) (width 0.3) (layer "F.Cu") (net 27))
 (via (at 72.55 121.5145) (size 0.8) (drill 0.4) (layers "F.Cu" "B.Cu") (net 27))
 (segment (start 89.7645 121.5145) (end 97.155 128.905) (width 0.3) (layer "B.Cu") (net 27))
 (segment (start 72.55 121.5145) (end 89.7645 121.5145) (width 0.3) (layer "B.Cu") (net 27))
 (segment (start 71.755 140.335) (end 61.115 129.695) (width 0.3) (layer "F.Cu") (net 24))
 (segment (start 96.52 150.495) (end 86.36 140.335) (width 0.3) (layer "F.Cu") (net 24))
 (segment (start 61.115 129.695) (end 61.115 125.19) (width 0.3) (layer "F.Cu") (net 24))
 (segment (start 86.36 140.335) (end 71.755 140.335) (width 0.3) (layer "F.Cu") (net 24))
 (segment (start 69.426666 150.495) (end 64.995 146.063334) (width 0.3) (layer "B.Cu") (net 11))
 (segment (start 64.995 126.53) (end 63.655 125.19) (width 0.3) (layer "B.Cu") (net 11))
 (segment (start 64.995 146.063334) (end 64.995 126.53) (width 0.3) (layer "B.Cu") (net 11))
 (segment (start 84.646701 114.743299) (end 78.895 120.495) (width 0.25) (layer "F.Cu") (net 10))
 (segment (start 89.175 114.743299) (end 84.646701 114.743299) (width 0.25) (layer "F.Cu") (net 10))
 (segment (start 78.895 117.63) (end 78.895 123.467665) (width 0.25) (layer "F.Cu") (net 10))
 (segment (start 76.008299 114.743299) (end 78.895 117.63) (width 0.25) (layer "F.Cu") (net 10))
 (segment (start 48.775 94.543299) (end 48.775 114.743299) (width 0.25) (layer "F.Cu") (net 10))
 (segment (start 68.975 114.743299) (end 76.008299 114.743299) (width 0.25) (layer "F.Cu") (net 10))
 (segment (start 78.895 123.467665) (end 78.895 125.19) (width 0.25) (layer "F.Cu") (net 10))
 (segment (start 78.895 120.495) (end 78.895 123.467665) (width 0.25) (layer "F.Cu") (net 10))
 (segment (start 68.975 114.743299) (end 48.775 114.743299) (width 0.25) (layer "F.Cu") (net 10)))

